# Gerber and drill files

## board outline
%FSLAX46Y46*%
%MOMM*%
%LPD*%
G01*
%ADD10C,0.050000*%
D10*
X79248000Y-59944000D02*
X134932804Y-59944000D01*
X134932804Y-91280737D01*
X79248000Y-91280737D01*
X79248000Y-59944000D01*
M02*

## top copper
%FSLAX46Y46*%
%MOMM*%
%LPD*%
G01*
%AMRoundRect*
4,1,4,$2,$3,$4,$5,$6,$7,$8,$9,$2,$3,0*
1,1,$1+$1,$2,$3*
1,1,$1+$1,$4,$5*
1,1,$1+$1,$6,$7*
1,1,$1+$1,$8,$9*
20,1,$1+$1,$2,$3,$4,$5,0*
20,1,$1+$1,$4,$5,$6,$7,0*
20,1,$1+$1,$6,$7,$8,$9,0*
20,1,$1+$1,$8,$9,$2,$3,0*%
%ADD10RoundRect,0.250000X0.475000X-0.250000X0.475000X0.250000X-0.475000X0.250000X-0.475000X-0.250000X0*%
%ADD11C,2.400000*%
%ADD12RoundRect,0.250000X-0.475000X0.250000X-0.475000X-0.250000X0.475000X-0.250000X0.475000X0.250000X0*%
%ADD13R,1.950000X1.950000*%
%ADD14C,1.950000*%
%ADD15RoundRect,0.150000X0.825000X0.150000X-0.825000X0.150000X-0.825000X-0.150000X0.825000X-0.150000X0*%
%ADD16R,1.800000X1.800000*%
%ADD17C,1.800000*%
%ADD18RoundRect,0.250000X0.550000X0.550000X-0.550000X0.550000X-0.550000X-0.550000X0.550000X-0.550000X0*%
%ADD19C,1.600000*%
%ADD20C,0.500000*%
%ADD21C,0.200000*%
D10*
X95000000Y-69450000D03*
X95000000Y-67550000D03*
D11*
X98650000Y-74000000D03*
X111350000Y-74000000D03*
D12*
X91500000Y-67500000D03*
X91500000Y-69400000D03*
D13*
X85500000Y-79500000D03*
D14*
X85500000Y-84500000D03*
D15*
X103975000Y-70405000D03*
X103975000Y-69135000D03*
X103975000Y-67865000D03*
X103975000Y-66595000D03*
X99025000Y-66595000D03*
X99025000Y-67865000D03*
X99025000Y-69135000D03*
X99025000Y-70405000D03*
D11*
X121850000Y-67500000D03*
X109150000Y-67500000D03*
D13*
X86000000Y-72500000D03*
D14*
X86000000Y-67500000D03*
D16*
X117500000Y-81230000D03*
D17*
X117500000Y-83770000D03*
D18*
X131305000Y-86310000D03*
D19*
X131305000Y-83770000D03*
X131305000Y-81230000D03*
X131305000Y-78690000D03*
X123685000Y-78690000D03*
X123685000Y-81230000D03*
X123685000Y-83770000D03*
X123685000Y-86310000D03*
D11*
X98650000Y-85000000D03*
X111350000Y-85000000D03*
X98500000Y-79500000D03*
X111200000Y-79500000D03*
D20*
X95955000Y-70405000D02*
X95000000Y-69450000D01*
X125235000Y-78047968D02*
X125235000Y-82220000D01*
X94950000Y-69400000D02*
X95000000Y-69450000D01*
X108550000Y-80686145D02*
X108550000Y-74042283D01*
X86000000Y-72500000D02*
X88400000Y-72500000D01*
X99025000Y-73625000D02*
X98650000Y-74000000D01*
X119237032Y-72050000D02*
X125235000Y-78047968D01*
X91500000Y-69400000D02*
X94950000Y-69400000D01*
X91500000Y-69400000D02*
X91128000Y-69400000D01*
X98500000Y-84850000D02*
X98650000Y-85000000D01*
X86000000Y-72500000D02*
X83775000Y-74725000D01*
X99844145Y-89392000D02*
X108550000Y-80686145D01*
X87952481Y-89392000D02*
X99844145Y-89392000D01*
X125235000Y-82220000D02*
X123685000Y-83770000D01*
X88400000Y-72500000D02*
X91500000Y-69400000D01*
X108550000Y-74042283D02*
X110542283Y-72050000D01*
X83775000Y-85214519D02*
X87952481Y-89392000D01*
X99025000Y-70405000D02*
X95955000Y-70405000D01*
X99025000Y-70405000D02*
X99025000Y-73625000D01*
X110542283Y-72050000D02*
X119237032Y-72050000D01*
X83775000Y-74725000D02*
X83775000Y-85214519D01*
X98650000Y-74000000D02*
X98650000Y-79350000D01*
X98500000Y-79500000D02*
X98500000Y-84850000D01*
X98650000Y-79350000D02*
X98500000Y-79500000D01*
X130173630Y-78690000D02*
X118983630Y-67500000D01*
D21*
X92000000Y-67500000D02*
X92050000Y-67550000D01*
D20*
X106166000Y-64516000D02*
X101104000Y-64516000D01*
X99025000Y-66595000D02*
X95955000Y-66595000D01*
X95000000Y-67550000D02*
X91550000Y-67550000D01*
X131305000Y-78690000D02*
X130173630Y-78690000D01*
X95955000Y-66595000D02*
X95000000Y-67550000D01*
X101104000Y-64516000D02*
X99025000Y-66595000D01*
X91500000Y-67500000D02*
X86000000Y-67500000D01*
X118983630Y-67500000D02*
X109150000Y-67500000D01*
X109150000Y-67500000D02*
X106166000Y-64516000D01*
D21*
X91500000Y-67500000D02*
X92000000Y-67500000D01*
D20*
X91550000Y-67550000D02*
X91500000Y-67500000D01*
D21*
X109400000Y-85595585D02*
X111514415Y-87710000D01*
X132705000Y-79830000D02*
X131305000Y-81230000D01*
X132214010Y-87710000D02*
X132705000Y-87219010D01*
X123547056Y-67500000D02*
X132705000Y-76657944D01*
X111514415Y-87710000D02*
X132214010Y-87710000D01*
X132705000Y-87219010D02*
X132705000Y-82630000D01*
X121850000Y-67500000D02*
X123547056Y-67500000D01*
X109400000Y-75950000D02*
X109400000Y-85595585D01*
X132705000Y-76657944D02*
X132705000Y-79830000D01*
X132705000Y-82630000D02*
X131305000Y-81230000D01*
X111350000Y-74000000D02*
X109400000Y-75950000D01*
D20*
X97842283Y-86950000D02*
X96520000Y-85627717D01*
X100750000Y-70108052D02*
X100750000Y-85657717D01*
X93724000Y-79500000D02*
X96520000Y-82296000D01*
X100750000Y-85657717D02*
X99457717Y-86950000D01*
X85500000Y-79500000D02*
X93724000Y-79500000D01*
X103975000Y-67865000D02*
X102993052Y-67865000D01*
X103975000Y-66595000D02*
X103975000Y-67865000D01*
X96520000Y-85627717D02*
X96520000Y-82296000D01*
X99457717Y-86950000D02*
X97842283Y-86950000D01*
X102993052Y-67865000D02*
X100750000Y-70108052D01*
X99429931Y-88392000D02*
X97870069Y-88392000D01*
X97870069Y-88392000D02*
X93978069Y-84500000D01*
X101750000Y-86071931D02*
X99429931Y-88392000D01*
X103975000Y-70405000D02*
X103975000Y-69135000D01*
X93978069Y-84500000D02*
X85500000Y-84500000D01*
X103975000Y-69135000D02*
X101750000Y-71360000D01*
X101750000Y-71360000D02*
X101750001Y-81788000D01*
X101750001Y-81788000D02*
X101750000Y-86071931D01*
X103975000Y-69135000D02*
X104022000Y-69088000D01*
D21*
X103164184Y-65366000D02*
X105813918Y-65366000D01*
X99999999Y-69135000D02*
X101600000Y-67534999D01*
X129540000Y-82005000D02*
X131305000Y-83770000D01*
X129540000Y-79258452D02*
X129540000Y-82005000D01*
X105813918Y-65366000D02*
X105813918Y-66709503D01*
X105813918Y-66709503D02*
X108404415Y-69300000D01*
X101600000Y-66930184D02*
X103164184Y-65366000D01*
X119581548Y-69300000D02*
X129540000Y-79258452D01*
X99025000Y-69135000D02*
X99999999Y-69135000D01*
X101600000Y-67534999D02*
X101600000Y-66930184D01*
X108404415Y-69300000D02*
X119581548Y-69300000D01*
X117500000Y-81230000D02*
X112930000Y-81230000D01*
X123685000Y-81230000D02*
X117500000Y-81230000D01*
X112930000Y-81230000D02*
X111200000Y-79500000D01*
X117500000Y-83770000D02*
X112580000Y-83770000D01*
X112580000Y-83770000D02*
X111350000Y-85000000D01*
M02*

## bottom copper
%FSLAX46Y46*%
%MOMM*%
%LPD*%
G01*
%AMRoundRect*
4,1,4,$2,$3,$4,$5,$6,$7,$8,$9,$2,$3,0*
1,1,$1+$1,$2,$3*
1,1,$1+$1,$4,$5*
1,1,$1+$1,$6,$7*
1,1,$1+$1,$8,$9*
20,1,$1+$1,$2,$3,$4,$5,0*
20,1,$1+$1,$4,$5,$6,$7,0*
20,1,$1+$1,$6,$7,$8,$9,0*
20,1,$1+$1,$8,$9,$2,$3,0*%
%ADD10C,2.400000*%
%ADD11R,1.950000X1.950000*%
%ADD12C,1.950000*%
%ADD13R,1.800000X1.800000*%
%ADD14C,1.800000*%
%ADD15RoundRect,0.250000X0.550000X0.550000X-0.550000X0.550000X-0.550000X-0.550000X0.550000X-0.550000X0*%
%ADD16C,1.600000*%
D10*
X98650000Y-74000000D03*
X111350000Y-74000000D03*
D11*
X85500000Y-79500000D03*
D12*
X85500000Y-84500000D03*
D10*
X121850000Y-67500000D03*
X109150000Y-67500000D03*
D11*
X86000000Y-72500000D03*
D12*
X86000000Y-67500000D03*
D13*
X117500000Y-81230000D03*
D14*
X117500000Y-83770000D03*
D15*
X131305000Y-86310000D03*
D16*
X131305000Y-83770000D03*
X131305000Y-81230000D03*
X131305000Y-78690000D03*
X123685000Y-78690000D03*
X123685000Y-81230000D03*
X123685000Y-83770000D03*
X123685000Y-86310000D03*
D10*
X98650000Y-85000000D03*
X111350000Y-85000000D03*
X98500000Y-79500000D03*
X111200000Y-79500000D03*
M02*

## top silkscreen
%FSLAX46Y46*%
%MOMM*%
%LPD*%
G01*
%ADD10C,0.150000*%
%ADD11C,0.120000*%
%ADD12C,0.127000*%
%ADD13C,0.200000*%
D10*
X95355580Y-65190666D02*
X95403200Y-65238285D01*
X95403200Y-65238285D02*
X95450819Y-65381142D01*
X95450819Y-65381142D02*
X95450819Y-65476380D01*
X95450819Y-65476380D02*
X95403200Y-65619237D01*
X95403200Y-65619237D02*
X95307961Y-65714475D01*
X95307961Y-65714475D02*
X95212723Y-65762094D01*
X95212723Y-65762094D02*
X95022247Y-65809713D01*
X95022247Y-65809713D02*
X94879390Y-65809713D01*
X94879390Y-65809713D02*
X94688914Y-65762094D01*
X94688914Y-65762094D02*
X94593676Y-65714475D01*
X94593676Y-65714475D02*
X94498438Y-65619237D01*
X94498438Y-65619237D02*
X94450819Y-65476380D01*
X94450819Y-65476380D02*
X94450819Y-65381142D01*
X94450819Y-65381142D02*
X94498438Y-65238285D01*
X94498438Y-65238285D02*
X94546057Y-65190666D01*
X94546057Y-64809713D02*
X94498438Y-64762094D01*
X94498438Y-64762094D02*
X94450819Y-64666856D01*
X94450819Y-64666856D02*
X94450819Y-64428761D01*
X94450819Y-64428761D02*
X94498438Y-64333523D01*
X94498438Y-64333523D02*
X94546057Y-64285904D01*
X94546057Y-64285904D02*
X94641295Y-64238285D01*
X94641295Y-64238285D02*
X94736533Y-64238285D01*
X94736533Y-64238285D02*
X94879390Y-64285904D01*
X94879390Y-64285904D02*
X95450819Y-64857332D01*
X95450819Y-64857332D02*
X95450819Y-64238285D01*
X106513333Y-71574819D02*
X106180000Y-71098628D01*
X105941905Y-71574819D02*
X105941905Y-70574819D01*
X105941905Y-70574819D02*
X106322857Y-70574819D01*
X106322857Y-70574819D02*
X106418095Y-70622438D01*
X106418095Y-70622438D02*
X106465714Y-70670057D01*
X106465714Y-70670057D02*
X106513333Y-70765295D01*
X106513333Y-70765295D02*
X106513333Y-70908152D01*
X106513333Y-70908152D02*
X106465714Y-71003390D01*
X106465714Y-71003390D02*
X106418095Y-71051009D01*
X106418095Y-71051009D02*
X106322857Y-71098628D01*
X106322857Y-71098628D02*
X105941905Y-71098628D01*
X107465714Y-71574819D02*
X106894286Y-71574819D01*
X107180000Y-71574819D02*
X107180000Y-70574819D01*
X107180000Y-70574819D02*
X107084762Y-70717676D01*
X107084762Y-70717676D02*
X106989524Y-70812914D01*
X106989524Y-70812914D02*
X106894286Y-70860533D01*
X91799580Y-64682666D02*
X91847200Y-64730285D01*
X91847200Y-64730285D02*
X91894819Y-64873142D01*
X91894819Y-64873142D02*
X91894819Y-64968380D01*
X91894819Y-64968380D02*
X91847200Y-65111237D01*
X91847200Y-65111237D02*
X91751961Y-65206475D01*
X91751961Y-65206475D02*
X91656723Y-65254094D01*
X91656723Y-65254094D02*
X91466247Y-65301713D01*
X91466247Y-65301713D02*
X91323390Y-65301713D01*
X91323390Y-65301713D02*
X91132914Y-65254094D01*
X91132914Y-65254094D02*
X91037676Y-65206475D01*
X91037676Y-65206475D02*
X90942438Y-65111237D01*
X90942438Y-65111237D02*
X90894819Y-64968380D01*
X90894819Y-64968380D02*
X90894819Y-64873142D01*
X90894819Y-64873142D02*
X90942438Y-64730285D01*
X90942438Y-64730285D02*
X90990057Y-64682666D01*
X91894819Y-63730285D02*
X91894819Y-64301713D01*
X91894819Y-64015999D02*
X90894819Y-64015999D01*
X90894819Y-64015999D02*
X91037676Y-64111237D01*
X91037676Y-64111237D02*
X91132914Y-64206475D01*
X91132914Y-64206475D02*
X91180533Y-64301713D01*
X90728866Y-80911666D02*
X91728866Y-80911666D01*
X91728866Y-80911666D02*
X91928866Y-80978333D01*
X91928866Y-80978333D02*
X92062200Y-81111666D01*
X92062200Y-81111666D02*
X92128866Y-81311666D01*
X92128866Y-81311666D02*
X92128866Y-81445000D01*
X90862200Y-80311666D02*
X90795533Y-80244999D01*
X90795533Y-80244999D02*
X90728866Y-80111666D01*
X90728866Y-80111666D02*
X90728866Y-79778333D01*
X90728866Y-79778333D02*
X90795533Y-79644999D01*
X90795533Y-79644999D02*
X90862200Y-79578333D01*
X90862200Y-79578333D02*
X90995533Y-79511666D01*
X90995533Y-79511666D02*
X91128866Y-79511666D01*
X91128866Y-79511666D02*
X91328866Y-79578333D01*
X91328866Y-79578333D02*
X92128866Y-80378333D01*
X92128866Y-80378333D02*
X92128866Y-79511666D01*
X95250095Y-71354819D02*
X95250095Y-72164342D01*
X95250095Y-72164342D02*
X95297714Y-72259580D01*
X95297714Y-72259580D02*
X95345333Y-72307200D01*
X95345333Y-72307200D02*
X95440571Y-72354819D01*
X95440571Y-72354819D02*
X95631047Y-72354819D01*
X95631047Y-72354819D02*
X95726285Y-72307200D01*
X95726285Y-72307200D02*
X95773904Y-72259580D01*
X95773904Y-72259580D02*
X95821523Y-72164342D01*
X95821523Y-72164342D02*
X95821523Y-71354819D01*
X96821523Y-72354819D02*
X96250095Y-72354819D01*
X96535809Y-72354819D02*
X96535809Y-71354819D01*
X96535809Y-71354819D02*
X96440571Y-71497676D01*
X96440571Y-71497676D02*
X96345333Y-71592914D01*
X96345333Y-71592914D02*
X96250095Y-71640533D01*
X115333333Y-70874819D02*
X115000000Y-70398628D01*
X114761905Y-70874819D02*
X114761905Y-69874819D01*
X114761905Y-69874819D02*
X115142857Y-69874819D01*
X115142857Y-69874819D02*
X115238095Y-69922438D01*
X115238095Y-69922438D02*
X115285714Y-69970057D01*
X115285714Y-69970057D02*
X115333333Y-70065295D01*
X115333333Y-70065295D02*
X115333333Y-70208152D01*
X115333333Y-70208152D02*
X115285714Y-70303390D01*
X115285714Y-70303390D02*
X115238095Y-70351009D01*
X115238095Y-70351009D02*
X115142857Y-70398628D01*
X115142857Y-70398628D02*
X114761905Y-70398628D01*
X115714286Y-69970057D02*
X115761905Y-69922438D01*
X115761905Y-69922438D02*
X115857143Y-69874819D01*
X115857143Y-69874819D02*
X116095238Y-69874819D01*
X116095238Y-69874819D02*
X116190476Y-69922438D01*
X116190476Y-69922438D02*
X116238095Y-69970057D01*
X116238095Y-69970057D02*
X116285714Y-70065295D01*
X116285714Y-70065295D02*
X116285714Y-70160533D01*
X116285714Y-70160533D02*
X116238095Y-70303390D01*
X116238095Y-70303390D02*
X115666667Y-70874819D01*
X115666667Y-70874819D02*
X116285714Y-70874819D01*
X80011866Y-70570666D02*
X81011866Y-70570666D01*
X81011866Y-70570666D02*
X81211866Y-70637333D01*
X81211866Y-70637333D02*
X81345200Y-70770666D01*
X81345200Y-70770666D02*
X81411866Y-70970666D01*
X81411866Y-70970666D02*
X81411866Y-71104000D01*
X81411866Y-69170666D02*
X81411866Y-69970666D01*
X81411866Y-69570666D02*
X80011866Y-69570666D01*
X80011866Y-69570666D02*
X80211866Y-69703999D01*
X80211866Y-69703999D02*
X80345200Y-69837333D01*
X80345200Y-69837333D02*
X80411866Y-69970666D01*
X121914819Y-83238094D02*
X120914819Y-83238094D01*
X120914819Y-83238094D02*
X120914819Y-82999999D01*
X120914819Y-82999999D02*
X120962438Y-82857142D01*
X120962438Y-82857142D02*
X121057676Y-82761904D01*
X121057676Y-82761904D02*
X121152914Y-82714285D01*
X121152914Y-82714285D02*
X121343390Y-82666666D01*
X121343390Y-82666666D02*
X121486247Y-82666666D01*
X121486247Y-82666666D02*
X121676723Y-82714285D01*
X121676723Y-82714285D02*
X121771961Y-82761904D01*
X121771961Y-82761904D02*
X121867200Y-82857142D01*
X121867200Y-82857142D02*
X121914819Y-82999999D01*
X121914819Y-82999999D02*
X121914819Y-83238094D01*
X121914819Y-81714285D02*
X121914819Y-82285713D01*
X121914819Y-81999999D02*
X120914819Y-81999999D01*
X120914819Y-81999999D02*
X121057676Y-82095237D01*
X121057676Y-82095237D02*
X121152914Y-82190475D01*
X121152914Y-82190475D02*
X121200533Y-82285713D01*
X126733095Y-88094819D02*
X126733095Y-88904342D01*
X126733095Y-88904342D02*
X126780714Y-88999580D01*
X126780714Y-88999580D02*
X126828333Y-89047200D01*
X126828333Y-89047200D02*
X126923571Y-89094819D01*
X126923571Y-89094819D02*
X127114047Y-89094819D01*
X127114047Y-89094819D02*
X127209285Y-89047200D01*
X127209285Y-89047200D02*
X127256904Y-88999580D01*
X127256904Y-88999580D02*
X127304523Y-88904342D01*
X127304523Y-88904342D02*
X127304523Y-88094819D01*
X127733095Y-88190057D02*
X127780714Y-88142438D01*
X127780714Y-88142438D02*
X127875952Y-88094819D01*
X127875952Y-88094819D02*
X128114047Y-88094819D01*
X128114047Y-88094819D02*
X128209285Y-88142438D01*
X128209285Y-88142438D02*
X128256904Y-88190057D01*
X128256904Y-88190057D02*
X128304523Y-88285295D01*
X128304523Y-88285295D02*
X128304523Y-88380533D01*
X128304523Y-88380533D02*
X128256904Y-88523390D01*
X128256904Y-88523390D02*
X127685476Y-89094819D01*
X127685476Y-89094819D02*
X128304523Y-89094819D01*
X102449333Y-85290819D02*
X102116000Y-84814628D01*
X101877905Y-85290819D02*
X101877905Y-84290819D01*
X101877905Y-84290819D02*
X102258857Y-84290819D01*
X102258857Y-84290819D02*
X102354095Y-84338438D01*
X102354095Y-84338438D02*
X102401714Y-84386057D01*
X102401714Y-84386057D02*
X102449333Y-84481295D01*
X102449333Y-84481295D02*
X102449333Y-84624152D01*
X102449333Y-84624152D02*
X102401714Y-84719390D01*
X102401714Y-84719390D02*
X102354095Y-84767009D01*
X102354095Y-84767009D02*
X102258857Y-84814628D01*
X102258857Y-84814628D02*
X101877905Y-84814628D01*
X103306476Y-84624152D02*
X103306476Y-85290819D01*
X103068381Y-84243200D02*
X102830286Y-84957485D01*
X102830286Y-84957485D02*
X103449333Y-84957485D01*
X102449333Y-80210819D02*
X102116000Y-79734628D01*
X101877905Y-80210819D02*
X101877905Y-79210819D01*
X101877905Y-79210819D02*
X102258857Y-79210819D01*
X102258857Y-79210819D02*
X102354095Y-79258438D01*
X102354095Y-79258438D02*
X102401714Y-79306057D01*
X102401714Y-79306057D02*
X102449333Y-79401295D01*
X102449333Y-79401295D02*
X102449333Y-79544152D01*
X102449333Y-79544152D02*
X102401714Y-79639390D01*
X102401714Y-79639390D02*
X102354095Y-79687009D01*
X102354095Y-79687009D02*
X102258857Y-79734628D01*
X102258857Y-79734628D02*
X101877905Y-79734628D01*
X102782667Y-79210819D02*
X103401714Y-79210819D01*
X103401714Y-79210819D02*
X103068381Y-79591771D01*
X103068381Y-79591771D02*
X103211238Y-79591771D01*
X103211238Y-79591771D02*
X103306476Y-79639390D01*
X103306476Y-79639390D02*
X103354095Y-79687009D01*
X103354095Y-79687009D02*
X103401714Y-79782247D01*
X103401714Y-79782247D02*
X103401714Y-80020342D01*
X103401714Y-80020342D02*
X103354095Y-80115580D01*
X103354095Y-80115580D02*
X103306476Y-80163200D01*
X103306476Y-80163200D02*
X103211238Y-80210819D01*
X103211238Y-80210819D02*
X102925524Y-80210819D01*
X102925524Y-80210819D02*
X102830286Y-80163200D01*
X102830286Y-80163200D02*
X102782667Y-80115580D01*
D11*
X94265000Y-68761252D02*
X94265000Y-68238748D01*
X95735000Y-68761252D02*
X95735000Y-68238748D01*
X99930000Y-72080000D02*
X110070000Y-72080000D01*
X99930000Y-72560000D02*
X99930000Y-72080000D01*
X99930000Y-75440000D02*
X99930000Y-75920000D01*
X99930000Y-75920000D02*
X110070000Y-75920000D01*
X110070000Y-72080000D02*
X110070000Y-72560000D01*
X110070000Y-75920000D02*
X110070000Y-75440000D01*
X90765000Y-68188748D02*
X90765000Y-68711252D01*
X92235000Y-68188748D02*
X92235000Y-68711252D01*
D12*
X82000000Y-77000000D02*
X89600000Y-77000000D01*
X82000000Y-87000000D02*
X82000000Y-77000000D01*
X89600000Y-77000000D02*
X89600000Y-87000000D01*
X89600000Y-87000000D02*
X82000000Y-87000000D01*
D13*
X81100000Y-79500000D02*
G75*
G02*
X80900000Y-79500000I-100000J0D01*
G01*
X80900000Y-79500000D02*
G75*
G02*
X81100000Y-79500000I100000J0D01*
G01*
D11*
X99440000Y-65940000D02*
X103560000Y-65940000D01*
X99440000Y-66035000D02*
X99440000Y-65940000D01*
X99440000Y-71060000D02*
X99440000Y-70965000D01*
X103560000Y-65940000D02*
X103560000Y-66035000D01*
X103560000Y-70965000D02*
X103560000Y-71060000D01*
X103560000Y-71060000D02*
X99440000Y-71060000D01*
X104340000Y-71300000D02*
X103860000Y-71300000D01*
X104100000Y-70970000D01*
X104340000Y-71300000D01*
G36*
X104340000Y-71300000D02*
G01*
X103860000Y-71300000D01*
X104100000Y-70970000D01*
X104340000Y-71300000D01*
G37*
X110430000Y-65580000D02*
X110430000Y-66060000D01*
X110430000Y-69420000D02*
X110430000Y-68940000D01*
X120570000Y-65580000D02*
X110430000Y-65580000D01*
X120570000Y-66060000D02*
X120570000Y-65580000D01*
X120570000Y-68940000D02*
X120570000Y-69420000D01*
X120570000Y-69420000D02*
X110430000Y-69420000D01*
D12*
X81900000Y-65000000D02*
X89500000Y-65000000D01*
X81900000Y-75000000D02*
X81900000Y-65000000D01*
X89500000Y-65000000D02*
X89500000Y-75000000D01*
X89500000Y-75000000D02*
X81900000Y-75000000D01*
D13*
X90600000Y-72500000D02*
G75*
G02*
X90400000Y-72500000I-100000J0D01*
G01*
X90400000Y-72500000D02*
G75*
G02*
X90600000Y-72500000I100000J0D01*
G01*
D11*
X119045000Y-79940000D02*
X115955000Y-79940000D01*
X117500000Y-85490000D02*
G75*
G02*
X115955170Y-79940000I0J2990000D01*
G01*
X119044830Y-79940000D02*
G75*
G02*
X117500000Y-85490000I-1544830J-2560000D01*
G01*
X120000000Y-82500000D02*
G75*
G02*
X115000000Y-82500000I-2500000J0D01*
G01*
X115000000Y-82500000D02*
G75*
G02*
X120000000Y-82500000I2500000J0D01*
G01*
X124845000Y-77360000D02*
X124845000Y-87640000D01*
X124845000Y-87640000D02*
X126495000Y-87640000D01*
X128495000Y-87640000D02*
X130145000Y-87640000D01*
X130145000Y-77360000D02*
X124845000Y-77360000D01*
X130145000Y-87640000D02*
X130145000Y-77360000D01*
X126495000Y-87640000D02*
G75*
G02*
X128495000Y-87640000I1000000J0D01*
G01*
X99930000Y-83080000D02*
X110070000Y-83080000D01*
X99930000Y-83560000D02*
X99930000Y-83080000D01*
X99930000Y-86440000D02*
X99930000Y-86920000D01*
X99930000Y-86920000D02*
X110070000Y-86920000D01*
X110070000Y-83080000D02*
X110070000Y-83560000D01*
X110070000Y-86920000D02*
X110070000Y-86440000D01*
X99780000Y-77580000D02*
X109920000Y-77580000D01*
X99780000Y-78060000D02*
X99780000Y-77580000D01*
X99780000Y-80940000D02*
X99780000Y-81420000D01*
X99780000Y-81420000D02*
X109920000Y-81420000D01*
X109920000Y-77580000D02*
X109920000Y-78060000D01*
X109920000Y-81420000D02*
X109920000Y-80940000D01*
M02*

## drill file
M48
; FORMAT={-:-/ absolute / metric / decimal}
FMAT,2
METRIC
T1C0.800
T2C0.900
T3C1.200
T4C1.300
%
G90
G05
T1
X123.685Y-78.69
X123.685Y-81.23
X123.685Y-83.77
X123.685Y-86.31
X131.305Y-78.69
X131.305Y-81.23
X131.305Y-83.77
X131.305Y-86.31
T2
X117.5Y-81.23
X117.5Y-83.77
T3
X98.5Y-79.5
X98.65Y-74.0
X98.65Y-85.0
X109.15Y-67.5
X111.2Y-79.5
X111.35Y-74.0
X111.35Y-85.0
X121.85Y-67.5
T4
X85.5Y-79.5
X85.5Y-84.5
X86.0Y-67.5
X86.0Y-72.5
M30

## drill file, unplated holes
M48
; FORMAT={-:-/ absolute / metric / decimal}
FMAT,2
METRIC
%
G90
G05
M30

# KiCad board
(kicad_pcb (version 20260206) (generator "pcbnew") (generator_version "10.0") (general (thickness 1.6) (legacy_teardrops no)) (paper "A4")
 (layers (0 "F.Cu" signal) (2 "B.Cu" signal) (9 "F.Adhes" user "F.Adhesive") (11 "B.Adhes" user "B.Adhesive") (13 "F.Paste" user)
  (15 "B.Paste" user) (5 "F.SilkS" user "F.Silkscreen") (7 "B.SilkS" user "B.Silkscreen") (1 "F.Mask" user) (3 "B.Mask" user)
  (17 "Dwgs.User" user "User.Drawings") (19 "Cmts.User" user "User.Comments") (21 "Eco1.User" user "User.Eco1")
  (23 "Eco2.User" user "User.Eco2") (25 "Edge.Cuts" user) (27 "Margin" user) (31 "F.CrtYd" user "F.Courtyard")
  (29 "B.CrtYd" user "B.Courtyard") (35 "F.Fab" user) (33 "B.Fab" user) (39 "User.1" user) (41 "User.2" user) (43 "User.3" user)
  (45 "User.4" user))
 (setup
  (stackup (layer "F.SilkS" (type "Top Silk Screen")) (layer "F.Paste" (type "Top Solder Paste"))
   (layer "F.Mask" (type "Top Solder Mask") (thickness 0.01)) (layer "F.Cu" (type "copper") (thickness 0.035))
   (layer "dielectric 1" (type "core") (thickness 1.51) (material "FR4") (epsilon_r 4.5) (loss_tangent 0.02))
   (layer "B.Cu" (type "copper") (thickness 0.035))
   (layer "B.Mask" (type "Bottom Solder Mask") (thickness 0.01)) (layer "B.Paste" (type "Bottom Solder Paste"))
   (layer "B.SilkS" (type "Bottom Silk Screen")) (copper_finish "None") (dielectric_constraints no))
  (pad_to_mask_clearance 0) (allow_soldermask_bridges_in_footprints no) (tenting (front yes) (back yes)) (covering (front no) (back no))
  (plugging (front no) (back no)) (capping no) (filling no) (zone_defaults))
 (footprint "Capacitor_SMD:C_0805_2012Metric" (layer "F.Cu") (at 95 68.5 90)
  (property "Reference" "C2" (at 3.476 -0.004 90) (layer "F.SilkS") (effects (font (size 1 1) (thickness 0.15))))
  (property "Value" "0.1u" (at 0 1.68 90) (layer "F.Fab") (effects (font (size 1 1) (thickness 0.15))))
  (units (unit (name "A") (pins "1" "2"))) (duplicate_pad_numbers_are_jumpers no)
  (fp_line (start -0.261252 -0.735) (end 0.261252 -0.735) (stroke (width 0.12) (type solid)) (layer "F.SilkS"))
  (fp_line (start -0.261252 0.735) (end 0.261252 0.735) (stroke (width 0.12) (type solid)) (layer "F.SilkS"))
  (pad "1" smd roundrect (at -0.95 0 90) (size 1 1.45) (layers "F.Cu" "F.Mask" "F.Paste") (roundrect_rratio 0.25) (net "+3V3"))
  (pad "2" smd roundrect (at 0.95 0 90) (size 1 1.45) (layers "F.Cu" "F.Mask" "F.Paste") (roundrect_rratio 0.25) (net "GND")))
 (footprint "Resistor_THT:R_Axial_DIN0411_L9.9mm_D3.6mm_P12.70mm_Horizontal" (layer "F.Cu") (at 98.65 74)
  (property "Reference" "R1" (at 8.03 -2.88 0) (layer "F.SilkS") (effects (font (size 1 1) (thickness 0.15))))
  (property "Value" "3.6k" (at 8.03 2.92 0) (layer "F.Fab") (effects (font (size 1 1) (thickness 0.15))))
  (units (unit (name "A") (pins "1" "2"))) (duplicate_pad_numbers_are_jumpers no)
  (fp_line (start 1.28 -1.92) (end 11.42 -1.92) (stroke (width 0.12) (type solid)) (layer "F.SilkS"))
  (fp_line (start 1.28 -1.44) (end 1.28 -1.92) (stroke (width 0.12) (type solid)) (layer "F.SilkS"))
  (fp_line (start 1.28 1.44) (end 1.28 1.92) (stroke (width 0.12) (type solid)) (layer "F.SilkS"))
  (fp_line (start 1.28 1.92) (end 11.42 1.92) (stroke (width 0.12) (type solid)) (layer "F.SilkS"))
  (fp_line (start 11.42 -1.92) (end 11.42 -1.44) (stroke (width 0.12) (type solid)) (layer "F.SilkS"))
  (fp_line (start 11.42 1.92) (end 11.42 1.44) (stroke (width 0.12) (type solid)) (layer "F.SilkS"))
  (pad "1" thru_hole circle (at 0 0) (size 2.4 2.4) (drill 1.2) (layers "*.Cu" "*.Mask") (remove_unused_layers no) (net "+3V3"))
  (pad "2" thru_hole circle (at 12.7 0) (size 2.4 2.4) (drill 1.2) (layers "*.Cu" "*.Mask") (remove_unused_layers no) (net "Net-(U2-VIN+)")))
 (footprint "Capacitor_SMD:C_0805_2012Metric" (layer "F.Cu") (at 91.5 68.45 -90)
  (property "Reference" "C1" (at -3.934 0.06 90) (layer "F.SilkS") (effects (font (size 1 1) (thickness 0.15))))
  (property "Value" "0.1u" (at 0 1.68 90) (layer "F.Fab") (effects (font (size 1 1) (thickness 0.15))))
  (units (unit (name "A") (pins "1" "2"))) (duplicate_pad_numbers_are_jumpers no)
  (fp_line (start -0.261252 0.735) (end 0.261252 0.735) (stroke (width 0.12) (type solid)) (layer "F.SilkS"))
  (fp_line (start -0.261252 -0.735) (end 0.261252 -0.735) (stroke (width 0.12) (type solid)) (layer "F.SilkS"))
  (pad "1" smd roundrect (at -0.95 0 270) (size 1 1.45) (layers "F.Cu" "F.Mask" "F.Paste") (roundrect_rratio 0.25) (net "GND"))
  (pad "2" smd roundrect (at 0.95 0 270) (size 1 1.45) (layers "F.Cu" "F.Mask" "F.Paste") (roundrect_rratio 0.25) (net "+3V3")))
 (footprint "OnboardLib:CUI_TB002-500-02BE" (layer "F.Cu") (at 85.5 79.5 -90)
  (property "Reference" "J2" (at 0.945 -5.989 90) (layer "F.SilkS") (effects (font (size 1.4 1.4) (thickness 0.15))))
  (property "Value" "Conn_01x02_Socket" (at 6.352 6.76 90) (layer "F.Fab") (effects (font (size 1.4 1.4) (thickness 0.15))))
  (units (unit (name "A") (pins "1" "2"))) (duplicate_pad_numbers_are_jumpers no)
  (fp_line (start -2.5 3.5) (end -2.5 -4.1) (stroke (width 0.127) (type solid)) (layer "F.SilkS"))
  (fp_line (start 7.5 3.5) (end -2.5 3.5) (stroke (width 0.127) (type solid)) (layer "F.SilkS"))
  (fp_line (start -2.5 -4.1) (end 7.5 -4.1) (stroke (width 0.127) (type solid)) (layer "F.SilkS"))
  (fp_line (start 7.5 -4.1) (end 7.5 3.5) (stroke (width 0.127) (type solid)) (layer "F.SilkS"))
  (fp_circle (center 0 4.5) (end 0.1 4.5) (stroke (width 0.2) (type solid)) (fill no) (layer "F.SilkS"))
  (pad "1" thru_hole rect (at 0 0 270) (size 1.95 1.95) (drill 1.3) (layers "*.Cu" "*.Mask") (remove_unused_layers no) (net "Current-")
   (solder_mask_margin 0.102))
  (pad "2" thru_hole circle (at 5 0 270) (size 1.95 1.95) (drill 1.3) (layers "*.Cu" "*.Mask") (remove_unused_layers no) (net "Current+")
   (solder_mask_margin 0.102)))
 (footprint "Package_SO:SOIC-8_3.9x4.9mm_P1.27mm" (layer "F.Cu") (at 101.5 68.5 180)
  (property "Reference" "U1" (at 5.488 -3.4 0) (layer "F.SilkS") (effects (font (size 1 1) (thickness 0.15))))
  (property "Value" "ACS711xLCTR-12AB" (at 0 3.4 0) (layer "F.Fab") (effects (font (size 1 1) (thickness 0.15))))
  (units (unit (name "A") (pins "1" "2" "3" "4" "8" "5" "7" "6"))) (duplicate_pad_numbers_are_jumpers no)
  (fp_line (start 2.06 2.56) (end -2.06 2.56) (stroke (width 0.12) (type solid)) (layer "F.SilkS"))
  (fp_line (start 2.06 2.465) (end 2.06 2.56) (stroke (width 0.12) (type solid)) (layer "F.SilkS"))
  (fp_line (start 2.06 -2.56) (end 2.06 -2.465) (stroke (width 0.12) (type solid)) (layer "F.SilkS"))
  (fp_line (start -2.06 2.56) (end -2.06 2.465) (stroke (width 0.12) (type solid)) (layer "F.SilkS"))
  (fp_line (start -2.06 -2.465) (end -2.06 -2.56) (stroke (width 0.12) (type solid)) (layer "F.SilkS"))
  (fp_line (start -2.06 -2.56) (end 2.06 -2.56) (stroke (width 0.12) (type solid)) (layer "F.SilkS"))
  (fp_poly (pts (xy -2.6 -2.47) (xy -2.84 -2.8) (xy -2.36 -2.8)) (stroke (width 0.12) (type solid)) (fill yes) (layer "F.SilkS"))
  (pad "1" smd roundrect (at -2.475 -1.905 180) (size 1.95 0.6) (layers "F.Cu" "F.Mask" "F.Paste") (roundrect_rratio 0.25) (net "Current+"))
  (pad "2" smd roundrect (at -2.475 -0.635 180) (size 1.95 0.6) (layers "F.Cu" "F.Mask" "F.Paste") (roundrect_rratio 0.25) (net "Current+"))
  (pad "3" smd roundrect (at -2.475 0.635 180) (size 1.95 0.6) (layers "F.Cu" "F.Mask" "F.Paste") (roundrect_rratio 0.25) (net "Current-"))
  (pad "4" smd roundrect (at -2.475 1.905 180) (size 1.95 0.6) (layers "F.Cu" "F.Mask" "F.Paste") (roundrect_rratio 0.25) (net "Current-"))
  (pad "5" smd roundrect (at 2.475 1.905 180) (size 1.95 0.6) (layers "F.Cu" "F.Mask" "F.Paste") (roundrect_rratio 0.25) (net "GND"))
  (pad "6" smd roundrect (at 2.475 0.635 180) (size 1.95 0.6) (layers "F.Cu" "F.Mask" "F.Paste") (roundrect_rratio 0.25)
   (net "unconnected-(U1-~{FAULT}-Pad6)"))
  (pad "7" smd roundrect (at 2.475 -0.635 180) (size 1.95 0.6) (layers "F.Cu" "F.Mask" "F.Paste") (roundrect_rratio 0.25)
   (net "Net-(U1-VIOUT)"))
  (pad "8" smd roundrect (at 2.475 -1.905 180) (size 1.95 0.6) (layers "F.Cu" "F.Mask" "F.Paste") (roundrect_rratio 0.25) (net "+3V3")))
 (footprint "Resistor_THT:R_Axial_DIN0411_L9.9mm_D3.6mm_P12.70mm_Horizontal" (layer "F.Cu") (at 121.85 67.5 180)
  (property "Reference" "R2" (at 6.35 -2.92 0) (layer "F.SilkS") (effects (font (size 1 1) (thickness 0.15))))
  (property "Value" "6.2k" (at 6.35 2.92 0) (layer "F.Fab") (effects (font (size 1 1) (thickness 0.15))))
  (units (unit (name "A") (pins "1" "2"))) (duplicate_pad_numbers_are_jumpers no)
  (fp_line (start 11.42 1.92) (end 11.42 1.44) (stroke (width 0.12) (type solid)) (layer "F.SilkS"))
  (fp_line (start 11.42 -1.92) (end 11.42 -1.44) (stroke (width 0.12) (type solid)) (layer "F.SilkS"))
  (fp_line (start 1.28 1.92) (end 11.42 1.92) (stroke (width 0.12) (type solid)) (layer "F.SilkS"))
  (fp_line (start 1.28 1.44) (end 1.28 1.92) (stroke (width 0.12) (type solid)) (layer "F.SilkS"))
  (fp_line (start 1.28 -1.44) (end 1.28 -1.92) (stroke (width 0.12) (type solid)) (layer "F.SilkS"))
  (fp_line (start 1.28 -1.92) (end 11.42 -1.92) (stroke (width 0.12) (type solid)) (layer "F.SilkS"))
  (pad "1" thru_hole circle (at 0 0 180) (size 2.4 2.4) (drill 1.2) (layers "*.Cu" "*.Mask") (remove_unused_layers no) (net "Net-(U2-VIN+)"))
  (pad "2" thru_hole circle (at 12.7 0 180) (size 2.4 2.4) (drill 1.2) (layers "*.Cu" "*.Mask") (remove_unused_layers no) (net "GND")))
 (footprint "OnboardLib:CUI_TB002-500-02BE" (layer "F.Cu") (at 86 72.5 90)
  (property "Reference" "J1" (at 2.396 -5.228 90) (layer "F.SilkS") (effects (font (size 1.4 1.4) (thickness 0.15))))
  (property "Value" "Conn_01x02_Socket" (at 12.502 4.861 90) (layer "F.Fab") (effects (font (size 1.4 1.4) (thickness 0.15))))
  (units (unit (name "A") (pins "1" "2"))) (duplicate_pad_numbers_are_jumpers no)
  (fp_line (start 7.5 -4.1) (end 7.5 3.5) (stroke (width 0.127) (type solid)) (layer "F.SilkS"))
  (fp_line (start -2.5 -4.1) (end 7.5 -4.1) (stroke (width 0.127) (type solid)) (layer "F.SilkS"))
  (fp_line (start 7.5 3.5) (end -2.5 3.5) (stroke (width 0.127) (type solid)) (layer "F.SilkS"))
  (fp_line (start -2.5 3.5) (end -2.5 -4.1) (stroke (width 0.127) (type solid)) (layer "F.SilkS"))
  (fp_circle (center 0 4.5) (end 0.1 4.5) (stroke (width 0.2) (type solid)) (fill no) (layer "F.SilkS"))
  (pad "1" thru_hole rect (at 0 0 90) (size 1.95 1.95) (drill 1.3) (layers "*.Cu" "*.Mask") (remove_unused_layers no) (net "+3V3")
   (solder_mask_margin 0.102))
  (pad "2" thru_hole circle (at 5 0 90) (size 1.95 1.95) (drill 1.3) (layers "*.Cu" "*.Mask") (remove_unused_layers no) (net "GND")
   (solder_mask_margin 0.102)))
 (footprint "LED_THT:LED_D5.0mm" (layer "F.Cu") (at 117.5 81.23 -90)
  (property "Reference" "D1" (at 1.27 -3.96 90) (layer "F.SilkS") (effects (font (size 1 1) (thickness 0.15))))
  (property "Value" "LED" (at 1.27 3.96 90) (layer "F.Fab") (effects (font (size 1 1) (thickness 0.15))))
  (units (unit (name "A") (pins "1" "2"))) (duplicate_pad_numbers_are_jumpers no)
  (fp_line (start -1.29 -1.545) (end -1.29 1.545) (stroke (width 0.12) (type solid)) (layer "F.SilkS"))
  (fp_arc (start 4.26 0) (mid 2.071779 2.880495) (end -1.29 1.54483) (stroke (width 0.12) (type solid)) (layer "F.SilkS"))
  (fp_arc (start -1.29 -1.54483) (mid 2.071779 -2.880495) (end 4.26 0) (stroke (width 0.12) (type solid)) (layer "F.SilkS"))
  (fp_circle (center 1.27 0) (end 3.77 0) (stroke (width 0.12) (type solid)) (fill no) (layer "F.SilkS"))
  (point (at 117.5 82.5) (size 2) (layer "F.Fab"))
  (pad "1" thru_hole rect (at 0 0 270) (size 1.8 1.8) (drill 0.9) (layers "*.Cu" "*.Mask") (remove_unused_layers no) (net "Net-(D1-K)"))
  (pad "2" thru_hole circle (at 2.54 0 270) (size 1.8 1.8) (drill 0.9) (layers "*.Cu" "*.Mask") (remove_unused_layers no) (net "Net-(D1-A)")))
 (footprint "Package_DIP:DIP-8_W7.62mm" (layer "F.Cu") (at 131.305 86.31 180)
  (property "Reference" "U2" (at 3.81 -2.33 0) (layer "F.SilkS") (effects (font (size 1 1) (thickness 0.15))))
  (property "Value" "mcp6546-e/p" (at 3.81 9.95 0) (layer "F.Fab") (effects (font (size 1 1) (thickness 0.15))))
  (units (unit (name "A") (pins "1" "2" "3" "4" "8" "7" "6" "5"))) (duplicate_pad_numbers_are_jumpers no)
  (fp_line (start 6.46 8.95) (end 6.46 -1.33) (stroke (width 0.12) (type solid)) (layer "F.SilkS"))
  (fp_line (start 6.46 -1.33) (end 4.81 -1.33) (stroke (width 0.12) (type solid)) (layer "F.SilkS"))
  (fp_line (start 2.81 -1.33) (end 1.16 -1.33) (stroke (width 0.12) (type solid)) (layer "F.SilkS"))
  (fp_line (start 1.16 8.95) (end 6.46 8.95) (stroke (width 0.12) (type solid)) (layer "F.SilkS"))
  (fp_line (start 1.16 -1.33) (end 1.16 8.95) (stroke (width 0.12) (type solid)) (layer "F.SilkS"))
  (fp_arc (start 4.81 -1.33) (mid 3.81 -0.33) (end 2.81 -1.33) (stroke (width 0.12) (type solid)) (layer "F.SilkS"))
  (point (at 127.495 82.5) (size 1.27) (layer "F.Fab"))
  (pad "1" thru_hole roundrect (at 0 0 180) (size 1.6 1.6) (drill 0.8) (layers "*.Cu" "*.Mask") (remove_unused_layers no)
   (roundrect_rratio 0.15625) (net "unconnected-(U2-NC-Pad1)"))
  (pad "2" thru_hole circle (at 0 2.54 180) (size 1.6 1.6) (drill 0.8) (layers "*.Cu" "*.Mask") (remove_unused_layers no)
   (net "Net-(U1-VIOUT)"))
  (pad "3" thru_hole circle (at 0 5.08 180) (size 1.6 1.6) (drill 0.8) (layers "*.Cu" "*.Mask") (remove_unused_layers no)
   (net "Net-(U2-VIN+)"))
  (pad "4" thru_hole circle (at 0 7.62 180) (size 1.6 1.6) (drill 0.8) (layers "*.Cu" "*.Mask") (remove_unused_layers no) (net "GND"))
  (pad "5" thru_hole circle (at 7.62 7.62 180) (size 1.6 1.6) (drill 0.8) (layers "*.Cu" "*.Mask") (remove_unused_layers no)
   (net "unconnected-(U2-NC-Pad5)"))
  (pad "6" thru_hole circle (at 7.62 5.08 180) (size 1.6 1.6) (drill 0.8) (layers "*.Cu" "*.Mask") (remove_unused_layers no)
   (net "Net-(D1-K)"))
  (pad "7" thru_hole circle (at 7.62 2.54 180) (size 1.6 1.6) (drill 0.8) (layers "*.Cu" "*.Mask") (remove_unused_layers no) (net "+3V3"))
  (pad "8" thru_hole circle (at 7.62 0 180) (size 1.6 1.6) (drill 0.8) (layers "*.Cu" "*.Mask") (remove_unused_layers no)
   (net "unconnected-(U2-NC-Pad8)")))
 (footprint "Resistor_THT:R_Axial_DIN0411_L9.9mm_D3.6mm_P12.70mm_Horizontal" (layer "F.Cu") (at 98.65 85)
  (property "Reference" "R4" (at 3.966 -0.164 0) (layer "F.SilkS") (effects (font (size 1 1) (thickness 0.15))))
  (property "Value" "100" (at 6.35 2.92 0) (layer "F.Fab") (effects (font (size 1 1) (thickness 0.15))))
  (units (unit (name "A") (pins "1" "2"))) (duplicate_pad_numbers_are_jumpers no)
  (fp_line (start 1.28 -1.92) (end 11.42 -1.92) (stroke (width 0.12) (type solid)) (layer "F.SilkS"))
  (fp_line (start 1.28 -1.44) (end 1.28 -1.92) (stroke (width 0.12) (type solid)) (layer "F.SilkS"))
  (fp_line (start 1.28 1.44) (end 1.28 1.92) (stroke (width 0.12) (type solid)) (layer "F.SilkS"))
  (fp_line (start 1.28 1.92) (end 11.42 1.92) (stroke (width 0.12) (type solid)) (layer "F.SilkS"))
  (fp_line (start 11.42 -1.92) (end 11.42 -1.44) (stroke (width 0.12) (type solid)) (layer "F.SilkS"))
  (fp_line (start 11.42 1.92) (end 11.42 1.44) (stroke (width 0.12) (type solid)) (layer "F.SilkS"))
  (pad "1" thru_hole circle (at 0 0) (size 2.4 2.4) (drill 1.2) (layers "*.Cu" "*.Mask") (remove_unused_layers no) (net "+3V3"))
  (pad "2" thru_hole circle (at 12.7 0) (size 2.4 2.4) (drill 1.2) (layers "*.Cu" "*.Mask") (remove_unused_layers no) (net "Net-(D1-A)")))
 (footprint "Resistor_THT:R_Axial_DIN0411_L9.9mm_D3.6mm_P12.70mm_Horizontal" (layer "F.Cu") (at 98.5 79.5)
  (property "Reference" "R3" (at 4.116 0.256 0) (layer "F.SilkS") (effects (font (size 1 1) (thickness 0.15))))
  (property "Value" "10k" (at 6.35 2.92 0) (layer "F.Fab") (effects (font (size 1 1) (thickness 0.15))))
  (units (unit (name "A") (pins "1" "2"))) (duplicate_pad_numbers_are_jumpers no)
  (fp_line (start 1.28 -1.92) (end 11.42 -1.92) (stroke (width 0.12) (type solid)) (layer "F.SilkS"))
  (fp_line (start 1.28 -1.44) (end 1.28 -1.92) (stroke (width 0.12) (type solid)) (layer "F.SilkS"))
  (fp_line (start 1.28 1.44) (end 1.28 1.92) (stroke (width 0.12) (type solid)) (layer "F.SilkS"))
  (fp_line (start 1.28 1.92) (end 11.42 1.92) (stroke (width 0.12) (type solid)) (layer "F.SilkS"))
  (fp_line (start 11.42 -1.92) (end 11.42 -1.44) (stroke (width 0.12) (type solid)) (layer "F.SilkS"))
  (fp_line (start 11.42 1.92) (end 11.42 1.44) (stroke (width 0.12) (type solid)) (layer "F.SilkS"))
  (pad "1" thru_hole circle (at 0 0) (size 2.4 2.4) (drill 1.2) (layers "*.Cu" "*.Mask") (remove_unused_layers no) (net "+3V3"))
  (pad "2" thru_hole circle (at 12.7 0) (size 2.4 2.4) (drill 1.2) (layers "*.Cu" "*.Mask") (remove_unused_layers no) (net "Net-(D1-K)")))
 (gr_rect (start 79.248 59.944) (end 134.932804 91.280737) (stroke (width 0.05) (type default)) (fill no) (layer "Edge.Cuts"))
 (segment (start 95.955 70.405) (end 95 69.45) (width 0.5) (layer "F.Cu") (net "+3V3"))
 (segment (start 125.235 78.047968) (end 125.235 82.22) (width 0.5) (layer "F.Cu") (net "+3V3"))
 (segment (start 94.95 69.4) (end 95 69.45) (width 0.5) (layer "F.Cu") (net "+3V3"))
 (segment (start 108.55 80.686145) (end 108.55 74.042283) (width 0.5) (layer "F.Cu") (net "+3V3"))
 (segment (start 86 72.5) (end 88.4 72.5) (width 0.5) (layer "F.Cu") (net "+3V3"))
 (segment (start 99.025 73.625) (end 98.65 74) (width 0.5) (layer "F.Cu") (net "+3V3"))
 (segment (start 119.237032 72.05) (end 125.235 78.047968) (width 0.5) (layer "F.Cu") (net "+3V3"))
 (segment (start 91.5 69.4) (end 94.95 69.4) (width 0.5) (layer "F.Cu") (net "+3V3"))
 (segment (start 91.5 69.4) (end 91.128 69.4) (width 0.5) (layer "F.Cu") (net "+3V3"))
 (segment (start 98.5 84.85) (end 98.65 85) (width 0.5) (layer "F.Cu") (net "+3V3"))
 (segment (start 86 72.5) (end 83.775 74.725) (width 0.5) (layer "F.Cu") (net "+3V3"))
 (segment (start 99.844145 89.392) (end 108.55 80.686145) (width 0.5) (layer "F.Cu") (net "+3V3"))
 (segment (start 87.952481 89.392) (end 99.844145 89.392) (width 0.5) (layer "F.Cu") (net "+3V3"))
 (segment (start 125.235 82.22) (end 123.685 83.77) (width 0.5) (layer "F.Cu") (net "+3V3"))
 (segment (start 88.4 72.5) (end 91.5 69.4) (width 0.5) (layer "F.Cu") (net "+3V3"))
 (segment (start 108.55 74.042283) (end 110.542283 72.05) (width 0.5) (layer "F.Cu") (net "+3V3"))
 (segment (start 83.775 85.214519) (end 87.952481 89.392) (width 0.5) (layer "F.Cu") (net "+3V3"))
 (segment (start 99.025 70.405) (end 95.955 70.405) (width 0.5) (layer "F.Cu") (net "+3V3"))
 (segment (start 99.025 70.405) (end 99.025 73.625) (width 0.5) (layer "F.Cu") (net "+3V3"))
 (segment (start 110.542283 72.05) (end 119.237032 72.05) (width 0.5) (layer "F.Cu") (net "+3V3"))
 (segment (start 83.775 74.725) (end 83.775 85.214519) (width 0.5) (layer "F.Cu") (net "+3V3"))
 (segment (start 98.65 74) (end 98.65 79.35) (width 0.5) (layer "F.Cu") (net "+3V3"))
 (segment (start 98.5 79.5) (end 98.5 84.85) (width 0.5) (layer "F.Cu") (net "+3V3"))
 (segment (start 98.65 79.35) (end 98.5 79.5) (width 0.5) (layer "F.Cu") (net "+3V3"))
 (segment (start 130.17363 78.69) (end 118.98363 67.5) (width 0.5) (layer "F.Cu") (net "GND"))
 (segment (start 92 67.5) (end 92.05 67.55) (width 0.2) (layer "F.Cu") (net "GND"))
 (segment (start 106.166 64.516) (end 101.104 64.516) (width 0.5) (layer "F.Cu") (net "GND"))
 (segment (start 99.025 66.595) (end 95.955 66.595) (width 0.5) (layer "F.Cu") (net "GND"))
 (segment (start 95 67.55) (end 91.55 67.55) (width 0.5) (layer "F.Cu") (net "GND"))
 (segment (start 131.305 78.69) (end 130.17363 78.69) (width 0.5) (layer "F.Cu") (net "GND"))
 (segment (start 95.955 66.595) (end 95 67.55) (width 0.5) (layer "F.Cu") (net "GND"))
 (segment (start 101.104 64.516) (end 99.025 66.595) (width 0.5) (layer "F.Cu") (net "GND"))
 (segment (start 91.5 67.5) (end 86 67.5) (width 0.5) (layer "F.Cu") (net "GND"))
 (segment (start 118.98363 67.5) (end 109.15 67.5) (width 0.5) (layer "F.Cu") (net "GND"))
 (segment (start 109.15 67.5) (end 106.166 64.516) (width 0.5) (layer "F.Cu") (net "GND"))
 (segment (start 91.5 67.5) (end 92 67.5) (width 0.2) (layer "F.Cu") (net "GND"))
 (segment (start 91.55 67.55) (end 91.5 67.5) (width 0.5) (layer "F.Cu") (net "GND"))
 (segment (start 109.4 85.595585) (end 111.514415 87.71) (width 0.2) (layer "F.Cu") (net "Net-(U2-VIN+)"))
 (segment (start 132.705 79.83) (end 131.305 81.23) (width 0.2) (layer "F.Cu") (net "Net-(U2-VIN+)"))
 (segment (start 132.21401 87.71) (end 132.705 87.21901) (width 0.2) (layer "F.Cu") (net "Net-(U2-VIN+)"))
 (segment (start 123.547056 67.5) (end 132.705 76.657944) (width 0.2) (layer "F.Cu") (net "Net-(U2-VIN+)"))
 (segment (start 111.514415 87.71) (end 132.21401 87.71) (width 0.2) (layer "F.Cu") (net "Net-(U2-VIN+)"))
 (segment (start 132.705 87.21901) (end 132.705 82.63) (width 0.2) (layer "F.Cu") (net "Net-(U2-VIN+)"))
 (segment (start 121.85 67.5) (end 123.547056 67.5) (width 0.2) (layer "F.Cu") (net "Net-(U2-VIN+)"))
 (segment (start 109.4 75.95) (end 109.4 85.595585) (width 0.2) (layer "F.Cu") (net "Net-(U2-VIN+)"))
 (segment (start 132.705 76.657944) (end 132.705 79.83) (width 0.2) (layer "F.Cu") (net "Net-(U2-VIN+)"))
 (segment (start 132.705 82.63) (end 131.305 81.23) (width 0.2) (layer "F.Cu") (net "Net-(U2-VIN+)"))
 (segment (start 111.35 74) (end 109.4 75.95) (width 0.2) (layer "F.Cu") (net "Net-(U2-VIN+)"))
 (segment (start 97.842283 86.95) (end 96.52 85.627717) (width 0.5) (layer "F.Cu") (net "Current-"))
 (segment (start 100.75 70.108052) (end 100.75 85.657717) (width 0.5) (layer "F.Cu") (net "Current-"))
 (segment (start 93.724 79.5) (end 96.52 82.296) (width 0.5) (layer "F.Cu") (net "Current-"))
 (segment (start 100.75 85.657717) (end 99.457717 86.95) (width 0.5) (layer "F.Cu") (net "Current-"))
 (segment (start 85.5 79.5) (end 93.724 79.5) (width 0.5) (layer "F.Cu") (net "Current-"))
 (segment (start 103.975 67.865) (end 102.993052 67.865) (width 0.5) (layer "F.Cu") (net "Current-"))
 (segment (start 103.975 66.595) (end 103.975 67.865) (width 0.5) (layer "F.Cu") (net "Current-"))
 (segment (start 96.52 85.627717) (end 96.52 82.296) (width 0.5) (layer "F.Cu") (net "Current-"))
 (segment (start 99.457717 86.95) (end 97.842283 86.95) (width 0.5) (layer "F.Cu") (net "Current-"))
 (segment (start 102.993052 67.865) (end 100.75 70.108052) (width 0.5) (layer "F.Cu") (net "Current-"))
 (segment (start 99.429931 88.392) (end 97.870069 88.392) (width 0.5) (layer "F.Cu") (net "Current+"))
 (segment (start 97.870069 88.392) (end 93.978069 84.5) (width 0.5) (layer "F.Cu") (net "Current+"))
 (segment (start 101.75 86.071931) (end 99.429931 88.392) (width 0.5) (layer "F.Cu") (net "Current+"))
 (segment (start 103.975 70.405) (end 103.975 69.135) (width 0.5) (layer "F.Cu") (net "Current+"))
 (segment (start 93.978069 84.5) (end 85.5 84.5) (width 0.5) (layer "F.Cu") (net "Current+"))
 (segment (start 103.975 69.135) (end 101.75 71.36) (width 0.5) (layer "F.Cu") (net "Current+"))
 (segment (start 101.75 71.36) (end 101.750001 81.788) (width 0.5) (layer "F.Cu") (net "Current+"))
 (segment (start 101.750001 81.788) (end 101.75 86.071931) (width 0.5) (layer "F.Cu") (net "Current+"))
 (segment (start 103.975 69.135) (end 104.022 69.088) (width 0.5) (layer "F.Cu") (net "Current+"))
 (segment (start 103.164184 65.366) (end 105.813918 65.366) (width 0.2) (layer "F.Cu") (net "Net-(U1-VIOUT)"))
 (segment (start 99.999999 69.135) (end 101.6 67.534999) (width 0.2) (layer "F.Cu") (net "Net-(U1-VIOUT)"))
 (segment (start 129.54 82.005) (end 131.305 83.77) (width 0.2) (layer "F.Cu") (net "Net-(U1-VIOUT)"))
 (segment (start 129.54 79.258452) (end 129.54 82.005) (width 0.2) (layer "F.Cu") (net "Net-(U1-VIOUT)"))
 (segment (start 105.813918 65.366) (end 105.813918 66.709503) (width 0.2) (layer "F.Cu") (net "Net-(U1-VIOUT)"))
 (segment (start 105.813918 66.709503) (end 108.404415 69.3) (width 0.2) (layer "F.Cu") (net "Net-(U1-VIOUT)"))
 (segment (start 101.6 66.930184) (end 103.164184 65.366) (width 0.2) (layer "F.Cu") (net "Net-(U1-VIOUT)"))
 (segment (start 119.581548 69.3) (end 129.54 79.258452) (width 0.2) (layer "F.Cu") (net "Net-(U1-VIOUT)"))
 (segment (start 99.025 69.135) (end 99.999999 69.135) (width 0.2) (layer "F.Cu") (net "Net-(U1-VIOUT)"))
 (segment (start 101.6 67.534999) (end 101.6 66.930184) (width 0.2) (layer "F.Cu") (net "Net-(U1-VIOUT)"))
 (segment (start 108.404415 69.3) (end 119.581548 69.3) (width 0.2) (layer "F.Cu") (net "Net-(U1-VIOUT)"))
 (segment (start 117.5 81.23) (end 112.93 81.23) (width 0.2) (layer "F.Cu") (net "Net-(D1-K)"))
 (segment (start 123.685 81.23) (end 117.5 81.23) (width 0.2) (layer "F.Cu") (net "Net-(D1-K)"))
 (segment (start 112.93 81.23) (end 111.2 79.5) (width 0.2) (layer "F.Cu") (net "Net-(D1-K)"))
 (segment (start 117.5 83.77) (end 112.58 83.77) (width 0.2) (layer "F.Cu") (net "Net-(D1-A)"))
 (segment (start 112.58 83.77) (end 111.35 85) (width 0.2) (layer "F.Cu") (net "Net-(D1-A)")))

